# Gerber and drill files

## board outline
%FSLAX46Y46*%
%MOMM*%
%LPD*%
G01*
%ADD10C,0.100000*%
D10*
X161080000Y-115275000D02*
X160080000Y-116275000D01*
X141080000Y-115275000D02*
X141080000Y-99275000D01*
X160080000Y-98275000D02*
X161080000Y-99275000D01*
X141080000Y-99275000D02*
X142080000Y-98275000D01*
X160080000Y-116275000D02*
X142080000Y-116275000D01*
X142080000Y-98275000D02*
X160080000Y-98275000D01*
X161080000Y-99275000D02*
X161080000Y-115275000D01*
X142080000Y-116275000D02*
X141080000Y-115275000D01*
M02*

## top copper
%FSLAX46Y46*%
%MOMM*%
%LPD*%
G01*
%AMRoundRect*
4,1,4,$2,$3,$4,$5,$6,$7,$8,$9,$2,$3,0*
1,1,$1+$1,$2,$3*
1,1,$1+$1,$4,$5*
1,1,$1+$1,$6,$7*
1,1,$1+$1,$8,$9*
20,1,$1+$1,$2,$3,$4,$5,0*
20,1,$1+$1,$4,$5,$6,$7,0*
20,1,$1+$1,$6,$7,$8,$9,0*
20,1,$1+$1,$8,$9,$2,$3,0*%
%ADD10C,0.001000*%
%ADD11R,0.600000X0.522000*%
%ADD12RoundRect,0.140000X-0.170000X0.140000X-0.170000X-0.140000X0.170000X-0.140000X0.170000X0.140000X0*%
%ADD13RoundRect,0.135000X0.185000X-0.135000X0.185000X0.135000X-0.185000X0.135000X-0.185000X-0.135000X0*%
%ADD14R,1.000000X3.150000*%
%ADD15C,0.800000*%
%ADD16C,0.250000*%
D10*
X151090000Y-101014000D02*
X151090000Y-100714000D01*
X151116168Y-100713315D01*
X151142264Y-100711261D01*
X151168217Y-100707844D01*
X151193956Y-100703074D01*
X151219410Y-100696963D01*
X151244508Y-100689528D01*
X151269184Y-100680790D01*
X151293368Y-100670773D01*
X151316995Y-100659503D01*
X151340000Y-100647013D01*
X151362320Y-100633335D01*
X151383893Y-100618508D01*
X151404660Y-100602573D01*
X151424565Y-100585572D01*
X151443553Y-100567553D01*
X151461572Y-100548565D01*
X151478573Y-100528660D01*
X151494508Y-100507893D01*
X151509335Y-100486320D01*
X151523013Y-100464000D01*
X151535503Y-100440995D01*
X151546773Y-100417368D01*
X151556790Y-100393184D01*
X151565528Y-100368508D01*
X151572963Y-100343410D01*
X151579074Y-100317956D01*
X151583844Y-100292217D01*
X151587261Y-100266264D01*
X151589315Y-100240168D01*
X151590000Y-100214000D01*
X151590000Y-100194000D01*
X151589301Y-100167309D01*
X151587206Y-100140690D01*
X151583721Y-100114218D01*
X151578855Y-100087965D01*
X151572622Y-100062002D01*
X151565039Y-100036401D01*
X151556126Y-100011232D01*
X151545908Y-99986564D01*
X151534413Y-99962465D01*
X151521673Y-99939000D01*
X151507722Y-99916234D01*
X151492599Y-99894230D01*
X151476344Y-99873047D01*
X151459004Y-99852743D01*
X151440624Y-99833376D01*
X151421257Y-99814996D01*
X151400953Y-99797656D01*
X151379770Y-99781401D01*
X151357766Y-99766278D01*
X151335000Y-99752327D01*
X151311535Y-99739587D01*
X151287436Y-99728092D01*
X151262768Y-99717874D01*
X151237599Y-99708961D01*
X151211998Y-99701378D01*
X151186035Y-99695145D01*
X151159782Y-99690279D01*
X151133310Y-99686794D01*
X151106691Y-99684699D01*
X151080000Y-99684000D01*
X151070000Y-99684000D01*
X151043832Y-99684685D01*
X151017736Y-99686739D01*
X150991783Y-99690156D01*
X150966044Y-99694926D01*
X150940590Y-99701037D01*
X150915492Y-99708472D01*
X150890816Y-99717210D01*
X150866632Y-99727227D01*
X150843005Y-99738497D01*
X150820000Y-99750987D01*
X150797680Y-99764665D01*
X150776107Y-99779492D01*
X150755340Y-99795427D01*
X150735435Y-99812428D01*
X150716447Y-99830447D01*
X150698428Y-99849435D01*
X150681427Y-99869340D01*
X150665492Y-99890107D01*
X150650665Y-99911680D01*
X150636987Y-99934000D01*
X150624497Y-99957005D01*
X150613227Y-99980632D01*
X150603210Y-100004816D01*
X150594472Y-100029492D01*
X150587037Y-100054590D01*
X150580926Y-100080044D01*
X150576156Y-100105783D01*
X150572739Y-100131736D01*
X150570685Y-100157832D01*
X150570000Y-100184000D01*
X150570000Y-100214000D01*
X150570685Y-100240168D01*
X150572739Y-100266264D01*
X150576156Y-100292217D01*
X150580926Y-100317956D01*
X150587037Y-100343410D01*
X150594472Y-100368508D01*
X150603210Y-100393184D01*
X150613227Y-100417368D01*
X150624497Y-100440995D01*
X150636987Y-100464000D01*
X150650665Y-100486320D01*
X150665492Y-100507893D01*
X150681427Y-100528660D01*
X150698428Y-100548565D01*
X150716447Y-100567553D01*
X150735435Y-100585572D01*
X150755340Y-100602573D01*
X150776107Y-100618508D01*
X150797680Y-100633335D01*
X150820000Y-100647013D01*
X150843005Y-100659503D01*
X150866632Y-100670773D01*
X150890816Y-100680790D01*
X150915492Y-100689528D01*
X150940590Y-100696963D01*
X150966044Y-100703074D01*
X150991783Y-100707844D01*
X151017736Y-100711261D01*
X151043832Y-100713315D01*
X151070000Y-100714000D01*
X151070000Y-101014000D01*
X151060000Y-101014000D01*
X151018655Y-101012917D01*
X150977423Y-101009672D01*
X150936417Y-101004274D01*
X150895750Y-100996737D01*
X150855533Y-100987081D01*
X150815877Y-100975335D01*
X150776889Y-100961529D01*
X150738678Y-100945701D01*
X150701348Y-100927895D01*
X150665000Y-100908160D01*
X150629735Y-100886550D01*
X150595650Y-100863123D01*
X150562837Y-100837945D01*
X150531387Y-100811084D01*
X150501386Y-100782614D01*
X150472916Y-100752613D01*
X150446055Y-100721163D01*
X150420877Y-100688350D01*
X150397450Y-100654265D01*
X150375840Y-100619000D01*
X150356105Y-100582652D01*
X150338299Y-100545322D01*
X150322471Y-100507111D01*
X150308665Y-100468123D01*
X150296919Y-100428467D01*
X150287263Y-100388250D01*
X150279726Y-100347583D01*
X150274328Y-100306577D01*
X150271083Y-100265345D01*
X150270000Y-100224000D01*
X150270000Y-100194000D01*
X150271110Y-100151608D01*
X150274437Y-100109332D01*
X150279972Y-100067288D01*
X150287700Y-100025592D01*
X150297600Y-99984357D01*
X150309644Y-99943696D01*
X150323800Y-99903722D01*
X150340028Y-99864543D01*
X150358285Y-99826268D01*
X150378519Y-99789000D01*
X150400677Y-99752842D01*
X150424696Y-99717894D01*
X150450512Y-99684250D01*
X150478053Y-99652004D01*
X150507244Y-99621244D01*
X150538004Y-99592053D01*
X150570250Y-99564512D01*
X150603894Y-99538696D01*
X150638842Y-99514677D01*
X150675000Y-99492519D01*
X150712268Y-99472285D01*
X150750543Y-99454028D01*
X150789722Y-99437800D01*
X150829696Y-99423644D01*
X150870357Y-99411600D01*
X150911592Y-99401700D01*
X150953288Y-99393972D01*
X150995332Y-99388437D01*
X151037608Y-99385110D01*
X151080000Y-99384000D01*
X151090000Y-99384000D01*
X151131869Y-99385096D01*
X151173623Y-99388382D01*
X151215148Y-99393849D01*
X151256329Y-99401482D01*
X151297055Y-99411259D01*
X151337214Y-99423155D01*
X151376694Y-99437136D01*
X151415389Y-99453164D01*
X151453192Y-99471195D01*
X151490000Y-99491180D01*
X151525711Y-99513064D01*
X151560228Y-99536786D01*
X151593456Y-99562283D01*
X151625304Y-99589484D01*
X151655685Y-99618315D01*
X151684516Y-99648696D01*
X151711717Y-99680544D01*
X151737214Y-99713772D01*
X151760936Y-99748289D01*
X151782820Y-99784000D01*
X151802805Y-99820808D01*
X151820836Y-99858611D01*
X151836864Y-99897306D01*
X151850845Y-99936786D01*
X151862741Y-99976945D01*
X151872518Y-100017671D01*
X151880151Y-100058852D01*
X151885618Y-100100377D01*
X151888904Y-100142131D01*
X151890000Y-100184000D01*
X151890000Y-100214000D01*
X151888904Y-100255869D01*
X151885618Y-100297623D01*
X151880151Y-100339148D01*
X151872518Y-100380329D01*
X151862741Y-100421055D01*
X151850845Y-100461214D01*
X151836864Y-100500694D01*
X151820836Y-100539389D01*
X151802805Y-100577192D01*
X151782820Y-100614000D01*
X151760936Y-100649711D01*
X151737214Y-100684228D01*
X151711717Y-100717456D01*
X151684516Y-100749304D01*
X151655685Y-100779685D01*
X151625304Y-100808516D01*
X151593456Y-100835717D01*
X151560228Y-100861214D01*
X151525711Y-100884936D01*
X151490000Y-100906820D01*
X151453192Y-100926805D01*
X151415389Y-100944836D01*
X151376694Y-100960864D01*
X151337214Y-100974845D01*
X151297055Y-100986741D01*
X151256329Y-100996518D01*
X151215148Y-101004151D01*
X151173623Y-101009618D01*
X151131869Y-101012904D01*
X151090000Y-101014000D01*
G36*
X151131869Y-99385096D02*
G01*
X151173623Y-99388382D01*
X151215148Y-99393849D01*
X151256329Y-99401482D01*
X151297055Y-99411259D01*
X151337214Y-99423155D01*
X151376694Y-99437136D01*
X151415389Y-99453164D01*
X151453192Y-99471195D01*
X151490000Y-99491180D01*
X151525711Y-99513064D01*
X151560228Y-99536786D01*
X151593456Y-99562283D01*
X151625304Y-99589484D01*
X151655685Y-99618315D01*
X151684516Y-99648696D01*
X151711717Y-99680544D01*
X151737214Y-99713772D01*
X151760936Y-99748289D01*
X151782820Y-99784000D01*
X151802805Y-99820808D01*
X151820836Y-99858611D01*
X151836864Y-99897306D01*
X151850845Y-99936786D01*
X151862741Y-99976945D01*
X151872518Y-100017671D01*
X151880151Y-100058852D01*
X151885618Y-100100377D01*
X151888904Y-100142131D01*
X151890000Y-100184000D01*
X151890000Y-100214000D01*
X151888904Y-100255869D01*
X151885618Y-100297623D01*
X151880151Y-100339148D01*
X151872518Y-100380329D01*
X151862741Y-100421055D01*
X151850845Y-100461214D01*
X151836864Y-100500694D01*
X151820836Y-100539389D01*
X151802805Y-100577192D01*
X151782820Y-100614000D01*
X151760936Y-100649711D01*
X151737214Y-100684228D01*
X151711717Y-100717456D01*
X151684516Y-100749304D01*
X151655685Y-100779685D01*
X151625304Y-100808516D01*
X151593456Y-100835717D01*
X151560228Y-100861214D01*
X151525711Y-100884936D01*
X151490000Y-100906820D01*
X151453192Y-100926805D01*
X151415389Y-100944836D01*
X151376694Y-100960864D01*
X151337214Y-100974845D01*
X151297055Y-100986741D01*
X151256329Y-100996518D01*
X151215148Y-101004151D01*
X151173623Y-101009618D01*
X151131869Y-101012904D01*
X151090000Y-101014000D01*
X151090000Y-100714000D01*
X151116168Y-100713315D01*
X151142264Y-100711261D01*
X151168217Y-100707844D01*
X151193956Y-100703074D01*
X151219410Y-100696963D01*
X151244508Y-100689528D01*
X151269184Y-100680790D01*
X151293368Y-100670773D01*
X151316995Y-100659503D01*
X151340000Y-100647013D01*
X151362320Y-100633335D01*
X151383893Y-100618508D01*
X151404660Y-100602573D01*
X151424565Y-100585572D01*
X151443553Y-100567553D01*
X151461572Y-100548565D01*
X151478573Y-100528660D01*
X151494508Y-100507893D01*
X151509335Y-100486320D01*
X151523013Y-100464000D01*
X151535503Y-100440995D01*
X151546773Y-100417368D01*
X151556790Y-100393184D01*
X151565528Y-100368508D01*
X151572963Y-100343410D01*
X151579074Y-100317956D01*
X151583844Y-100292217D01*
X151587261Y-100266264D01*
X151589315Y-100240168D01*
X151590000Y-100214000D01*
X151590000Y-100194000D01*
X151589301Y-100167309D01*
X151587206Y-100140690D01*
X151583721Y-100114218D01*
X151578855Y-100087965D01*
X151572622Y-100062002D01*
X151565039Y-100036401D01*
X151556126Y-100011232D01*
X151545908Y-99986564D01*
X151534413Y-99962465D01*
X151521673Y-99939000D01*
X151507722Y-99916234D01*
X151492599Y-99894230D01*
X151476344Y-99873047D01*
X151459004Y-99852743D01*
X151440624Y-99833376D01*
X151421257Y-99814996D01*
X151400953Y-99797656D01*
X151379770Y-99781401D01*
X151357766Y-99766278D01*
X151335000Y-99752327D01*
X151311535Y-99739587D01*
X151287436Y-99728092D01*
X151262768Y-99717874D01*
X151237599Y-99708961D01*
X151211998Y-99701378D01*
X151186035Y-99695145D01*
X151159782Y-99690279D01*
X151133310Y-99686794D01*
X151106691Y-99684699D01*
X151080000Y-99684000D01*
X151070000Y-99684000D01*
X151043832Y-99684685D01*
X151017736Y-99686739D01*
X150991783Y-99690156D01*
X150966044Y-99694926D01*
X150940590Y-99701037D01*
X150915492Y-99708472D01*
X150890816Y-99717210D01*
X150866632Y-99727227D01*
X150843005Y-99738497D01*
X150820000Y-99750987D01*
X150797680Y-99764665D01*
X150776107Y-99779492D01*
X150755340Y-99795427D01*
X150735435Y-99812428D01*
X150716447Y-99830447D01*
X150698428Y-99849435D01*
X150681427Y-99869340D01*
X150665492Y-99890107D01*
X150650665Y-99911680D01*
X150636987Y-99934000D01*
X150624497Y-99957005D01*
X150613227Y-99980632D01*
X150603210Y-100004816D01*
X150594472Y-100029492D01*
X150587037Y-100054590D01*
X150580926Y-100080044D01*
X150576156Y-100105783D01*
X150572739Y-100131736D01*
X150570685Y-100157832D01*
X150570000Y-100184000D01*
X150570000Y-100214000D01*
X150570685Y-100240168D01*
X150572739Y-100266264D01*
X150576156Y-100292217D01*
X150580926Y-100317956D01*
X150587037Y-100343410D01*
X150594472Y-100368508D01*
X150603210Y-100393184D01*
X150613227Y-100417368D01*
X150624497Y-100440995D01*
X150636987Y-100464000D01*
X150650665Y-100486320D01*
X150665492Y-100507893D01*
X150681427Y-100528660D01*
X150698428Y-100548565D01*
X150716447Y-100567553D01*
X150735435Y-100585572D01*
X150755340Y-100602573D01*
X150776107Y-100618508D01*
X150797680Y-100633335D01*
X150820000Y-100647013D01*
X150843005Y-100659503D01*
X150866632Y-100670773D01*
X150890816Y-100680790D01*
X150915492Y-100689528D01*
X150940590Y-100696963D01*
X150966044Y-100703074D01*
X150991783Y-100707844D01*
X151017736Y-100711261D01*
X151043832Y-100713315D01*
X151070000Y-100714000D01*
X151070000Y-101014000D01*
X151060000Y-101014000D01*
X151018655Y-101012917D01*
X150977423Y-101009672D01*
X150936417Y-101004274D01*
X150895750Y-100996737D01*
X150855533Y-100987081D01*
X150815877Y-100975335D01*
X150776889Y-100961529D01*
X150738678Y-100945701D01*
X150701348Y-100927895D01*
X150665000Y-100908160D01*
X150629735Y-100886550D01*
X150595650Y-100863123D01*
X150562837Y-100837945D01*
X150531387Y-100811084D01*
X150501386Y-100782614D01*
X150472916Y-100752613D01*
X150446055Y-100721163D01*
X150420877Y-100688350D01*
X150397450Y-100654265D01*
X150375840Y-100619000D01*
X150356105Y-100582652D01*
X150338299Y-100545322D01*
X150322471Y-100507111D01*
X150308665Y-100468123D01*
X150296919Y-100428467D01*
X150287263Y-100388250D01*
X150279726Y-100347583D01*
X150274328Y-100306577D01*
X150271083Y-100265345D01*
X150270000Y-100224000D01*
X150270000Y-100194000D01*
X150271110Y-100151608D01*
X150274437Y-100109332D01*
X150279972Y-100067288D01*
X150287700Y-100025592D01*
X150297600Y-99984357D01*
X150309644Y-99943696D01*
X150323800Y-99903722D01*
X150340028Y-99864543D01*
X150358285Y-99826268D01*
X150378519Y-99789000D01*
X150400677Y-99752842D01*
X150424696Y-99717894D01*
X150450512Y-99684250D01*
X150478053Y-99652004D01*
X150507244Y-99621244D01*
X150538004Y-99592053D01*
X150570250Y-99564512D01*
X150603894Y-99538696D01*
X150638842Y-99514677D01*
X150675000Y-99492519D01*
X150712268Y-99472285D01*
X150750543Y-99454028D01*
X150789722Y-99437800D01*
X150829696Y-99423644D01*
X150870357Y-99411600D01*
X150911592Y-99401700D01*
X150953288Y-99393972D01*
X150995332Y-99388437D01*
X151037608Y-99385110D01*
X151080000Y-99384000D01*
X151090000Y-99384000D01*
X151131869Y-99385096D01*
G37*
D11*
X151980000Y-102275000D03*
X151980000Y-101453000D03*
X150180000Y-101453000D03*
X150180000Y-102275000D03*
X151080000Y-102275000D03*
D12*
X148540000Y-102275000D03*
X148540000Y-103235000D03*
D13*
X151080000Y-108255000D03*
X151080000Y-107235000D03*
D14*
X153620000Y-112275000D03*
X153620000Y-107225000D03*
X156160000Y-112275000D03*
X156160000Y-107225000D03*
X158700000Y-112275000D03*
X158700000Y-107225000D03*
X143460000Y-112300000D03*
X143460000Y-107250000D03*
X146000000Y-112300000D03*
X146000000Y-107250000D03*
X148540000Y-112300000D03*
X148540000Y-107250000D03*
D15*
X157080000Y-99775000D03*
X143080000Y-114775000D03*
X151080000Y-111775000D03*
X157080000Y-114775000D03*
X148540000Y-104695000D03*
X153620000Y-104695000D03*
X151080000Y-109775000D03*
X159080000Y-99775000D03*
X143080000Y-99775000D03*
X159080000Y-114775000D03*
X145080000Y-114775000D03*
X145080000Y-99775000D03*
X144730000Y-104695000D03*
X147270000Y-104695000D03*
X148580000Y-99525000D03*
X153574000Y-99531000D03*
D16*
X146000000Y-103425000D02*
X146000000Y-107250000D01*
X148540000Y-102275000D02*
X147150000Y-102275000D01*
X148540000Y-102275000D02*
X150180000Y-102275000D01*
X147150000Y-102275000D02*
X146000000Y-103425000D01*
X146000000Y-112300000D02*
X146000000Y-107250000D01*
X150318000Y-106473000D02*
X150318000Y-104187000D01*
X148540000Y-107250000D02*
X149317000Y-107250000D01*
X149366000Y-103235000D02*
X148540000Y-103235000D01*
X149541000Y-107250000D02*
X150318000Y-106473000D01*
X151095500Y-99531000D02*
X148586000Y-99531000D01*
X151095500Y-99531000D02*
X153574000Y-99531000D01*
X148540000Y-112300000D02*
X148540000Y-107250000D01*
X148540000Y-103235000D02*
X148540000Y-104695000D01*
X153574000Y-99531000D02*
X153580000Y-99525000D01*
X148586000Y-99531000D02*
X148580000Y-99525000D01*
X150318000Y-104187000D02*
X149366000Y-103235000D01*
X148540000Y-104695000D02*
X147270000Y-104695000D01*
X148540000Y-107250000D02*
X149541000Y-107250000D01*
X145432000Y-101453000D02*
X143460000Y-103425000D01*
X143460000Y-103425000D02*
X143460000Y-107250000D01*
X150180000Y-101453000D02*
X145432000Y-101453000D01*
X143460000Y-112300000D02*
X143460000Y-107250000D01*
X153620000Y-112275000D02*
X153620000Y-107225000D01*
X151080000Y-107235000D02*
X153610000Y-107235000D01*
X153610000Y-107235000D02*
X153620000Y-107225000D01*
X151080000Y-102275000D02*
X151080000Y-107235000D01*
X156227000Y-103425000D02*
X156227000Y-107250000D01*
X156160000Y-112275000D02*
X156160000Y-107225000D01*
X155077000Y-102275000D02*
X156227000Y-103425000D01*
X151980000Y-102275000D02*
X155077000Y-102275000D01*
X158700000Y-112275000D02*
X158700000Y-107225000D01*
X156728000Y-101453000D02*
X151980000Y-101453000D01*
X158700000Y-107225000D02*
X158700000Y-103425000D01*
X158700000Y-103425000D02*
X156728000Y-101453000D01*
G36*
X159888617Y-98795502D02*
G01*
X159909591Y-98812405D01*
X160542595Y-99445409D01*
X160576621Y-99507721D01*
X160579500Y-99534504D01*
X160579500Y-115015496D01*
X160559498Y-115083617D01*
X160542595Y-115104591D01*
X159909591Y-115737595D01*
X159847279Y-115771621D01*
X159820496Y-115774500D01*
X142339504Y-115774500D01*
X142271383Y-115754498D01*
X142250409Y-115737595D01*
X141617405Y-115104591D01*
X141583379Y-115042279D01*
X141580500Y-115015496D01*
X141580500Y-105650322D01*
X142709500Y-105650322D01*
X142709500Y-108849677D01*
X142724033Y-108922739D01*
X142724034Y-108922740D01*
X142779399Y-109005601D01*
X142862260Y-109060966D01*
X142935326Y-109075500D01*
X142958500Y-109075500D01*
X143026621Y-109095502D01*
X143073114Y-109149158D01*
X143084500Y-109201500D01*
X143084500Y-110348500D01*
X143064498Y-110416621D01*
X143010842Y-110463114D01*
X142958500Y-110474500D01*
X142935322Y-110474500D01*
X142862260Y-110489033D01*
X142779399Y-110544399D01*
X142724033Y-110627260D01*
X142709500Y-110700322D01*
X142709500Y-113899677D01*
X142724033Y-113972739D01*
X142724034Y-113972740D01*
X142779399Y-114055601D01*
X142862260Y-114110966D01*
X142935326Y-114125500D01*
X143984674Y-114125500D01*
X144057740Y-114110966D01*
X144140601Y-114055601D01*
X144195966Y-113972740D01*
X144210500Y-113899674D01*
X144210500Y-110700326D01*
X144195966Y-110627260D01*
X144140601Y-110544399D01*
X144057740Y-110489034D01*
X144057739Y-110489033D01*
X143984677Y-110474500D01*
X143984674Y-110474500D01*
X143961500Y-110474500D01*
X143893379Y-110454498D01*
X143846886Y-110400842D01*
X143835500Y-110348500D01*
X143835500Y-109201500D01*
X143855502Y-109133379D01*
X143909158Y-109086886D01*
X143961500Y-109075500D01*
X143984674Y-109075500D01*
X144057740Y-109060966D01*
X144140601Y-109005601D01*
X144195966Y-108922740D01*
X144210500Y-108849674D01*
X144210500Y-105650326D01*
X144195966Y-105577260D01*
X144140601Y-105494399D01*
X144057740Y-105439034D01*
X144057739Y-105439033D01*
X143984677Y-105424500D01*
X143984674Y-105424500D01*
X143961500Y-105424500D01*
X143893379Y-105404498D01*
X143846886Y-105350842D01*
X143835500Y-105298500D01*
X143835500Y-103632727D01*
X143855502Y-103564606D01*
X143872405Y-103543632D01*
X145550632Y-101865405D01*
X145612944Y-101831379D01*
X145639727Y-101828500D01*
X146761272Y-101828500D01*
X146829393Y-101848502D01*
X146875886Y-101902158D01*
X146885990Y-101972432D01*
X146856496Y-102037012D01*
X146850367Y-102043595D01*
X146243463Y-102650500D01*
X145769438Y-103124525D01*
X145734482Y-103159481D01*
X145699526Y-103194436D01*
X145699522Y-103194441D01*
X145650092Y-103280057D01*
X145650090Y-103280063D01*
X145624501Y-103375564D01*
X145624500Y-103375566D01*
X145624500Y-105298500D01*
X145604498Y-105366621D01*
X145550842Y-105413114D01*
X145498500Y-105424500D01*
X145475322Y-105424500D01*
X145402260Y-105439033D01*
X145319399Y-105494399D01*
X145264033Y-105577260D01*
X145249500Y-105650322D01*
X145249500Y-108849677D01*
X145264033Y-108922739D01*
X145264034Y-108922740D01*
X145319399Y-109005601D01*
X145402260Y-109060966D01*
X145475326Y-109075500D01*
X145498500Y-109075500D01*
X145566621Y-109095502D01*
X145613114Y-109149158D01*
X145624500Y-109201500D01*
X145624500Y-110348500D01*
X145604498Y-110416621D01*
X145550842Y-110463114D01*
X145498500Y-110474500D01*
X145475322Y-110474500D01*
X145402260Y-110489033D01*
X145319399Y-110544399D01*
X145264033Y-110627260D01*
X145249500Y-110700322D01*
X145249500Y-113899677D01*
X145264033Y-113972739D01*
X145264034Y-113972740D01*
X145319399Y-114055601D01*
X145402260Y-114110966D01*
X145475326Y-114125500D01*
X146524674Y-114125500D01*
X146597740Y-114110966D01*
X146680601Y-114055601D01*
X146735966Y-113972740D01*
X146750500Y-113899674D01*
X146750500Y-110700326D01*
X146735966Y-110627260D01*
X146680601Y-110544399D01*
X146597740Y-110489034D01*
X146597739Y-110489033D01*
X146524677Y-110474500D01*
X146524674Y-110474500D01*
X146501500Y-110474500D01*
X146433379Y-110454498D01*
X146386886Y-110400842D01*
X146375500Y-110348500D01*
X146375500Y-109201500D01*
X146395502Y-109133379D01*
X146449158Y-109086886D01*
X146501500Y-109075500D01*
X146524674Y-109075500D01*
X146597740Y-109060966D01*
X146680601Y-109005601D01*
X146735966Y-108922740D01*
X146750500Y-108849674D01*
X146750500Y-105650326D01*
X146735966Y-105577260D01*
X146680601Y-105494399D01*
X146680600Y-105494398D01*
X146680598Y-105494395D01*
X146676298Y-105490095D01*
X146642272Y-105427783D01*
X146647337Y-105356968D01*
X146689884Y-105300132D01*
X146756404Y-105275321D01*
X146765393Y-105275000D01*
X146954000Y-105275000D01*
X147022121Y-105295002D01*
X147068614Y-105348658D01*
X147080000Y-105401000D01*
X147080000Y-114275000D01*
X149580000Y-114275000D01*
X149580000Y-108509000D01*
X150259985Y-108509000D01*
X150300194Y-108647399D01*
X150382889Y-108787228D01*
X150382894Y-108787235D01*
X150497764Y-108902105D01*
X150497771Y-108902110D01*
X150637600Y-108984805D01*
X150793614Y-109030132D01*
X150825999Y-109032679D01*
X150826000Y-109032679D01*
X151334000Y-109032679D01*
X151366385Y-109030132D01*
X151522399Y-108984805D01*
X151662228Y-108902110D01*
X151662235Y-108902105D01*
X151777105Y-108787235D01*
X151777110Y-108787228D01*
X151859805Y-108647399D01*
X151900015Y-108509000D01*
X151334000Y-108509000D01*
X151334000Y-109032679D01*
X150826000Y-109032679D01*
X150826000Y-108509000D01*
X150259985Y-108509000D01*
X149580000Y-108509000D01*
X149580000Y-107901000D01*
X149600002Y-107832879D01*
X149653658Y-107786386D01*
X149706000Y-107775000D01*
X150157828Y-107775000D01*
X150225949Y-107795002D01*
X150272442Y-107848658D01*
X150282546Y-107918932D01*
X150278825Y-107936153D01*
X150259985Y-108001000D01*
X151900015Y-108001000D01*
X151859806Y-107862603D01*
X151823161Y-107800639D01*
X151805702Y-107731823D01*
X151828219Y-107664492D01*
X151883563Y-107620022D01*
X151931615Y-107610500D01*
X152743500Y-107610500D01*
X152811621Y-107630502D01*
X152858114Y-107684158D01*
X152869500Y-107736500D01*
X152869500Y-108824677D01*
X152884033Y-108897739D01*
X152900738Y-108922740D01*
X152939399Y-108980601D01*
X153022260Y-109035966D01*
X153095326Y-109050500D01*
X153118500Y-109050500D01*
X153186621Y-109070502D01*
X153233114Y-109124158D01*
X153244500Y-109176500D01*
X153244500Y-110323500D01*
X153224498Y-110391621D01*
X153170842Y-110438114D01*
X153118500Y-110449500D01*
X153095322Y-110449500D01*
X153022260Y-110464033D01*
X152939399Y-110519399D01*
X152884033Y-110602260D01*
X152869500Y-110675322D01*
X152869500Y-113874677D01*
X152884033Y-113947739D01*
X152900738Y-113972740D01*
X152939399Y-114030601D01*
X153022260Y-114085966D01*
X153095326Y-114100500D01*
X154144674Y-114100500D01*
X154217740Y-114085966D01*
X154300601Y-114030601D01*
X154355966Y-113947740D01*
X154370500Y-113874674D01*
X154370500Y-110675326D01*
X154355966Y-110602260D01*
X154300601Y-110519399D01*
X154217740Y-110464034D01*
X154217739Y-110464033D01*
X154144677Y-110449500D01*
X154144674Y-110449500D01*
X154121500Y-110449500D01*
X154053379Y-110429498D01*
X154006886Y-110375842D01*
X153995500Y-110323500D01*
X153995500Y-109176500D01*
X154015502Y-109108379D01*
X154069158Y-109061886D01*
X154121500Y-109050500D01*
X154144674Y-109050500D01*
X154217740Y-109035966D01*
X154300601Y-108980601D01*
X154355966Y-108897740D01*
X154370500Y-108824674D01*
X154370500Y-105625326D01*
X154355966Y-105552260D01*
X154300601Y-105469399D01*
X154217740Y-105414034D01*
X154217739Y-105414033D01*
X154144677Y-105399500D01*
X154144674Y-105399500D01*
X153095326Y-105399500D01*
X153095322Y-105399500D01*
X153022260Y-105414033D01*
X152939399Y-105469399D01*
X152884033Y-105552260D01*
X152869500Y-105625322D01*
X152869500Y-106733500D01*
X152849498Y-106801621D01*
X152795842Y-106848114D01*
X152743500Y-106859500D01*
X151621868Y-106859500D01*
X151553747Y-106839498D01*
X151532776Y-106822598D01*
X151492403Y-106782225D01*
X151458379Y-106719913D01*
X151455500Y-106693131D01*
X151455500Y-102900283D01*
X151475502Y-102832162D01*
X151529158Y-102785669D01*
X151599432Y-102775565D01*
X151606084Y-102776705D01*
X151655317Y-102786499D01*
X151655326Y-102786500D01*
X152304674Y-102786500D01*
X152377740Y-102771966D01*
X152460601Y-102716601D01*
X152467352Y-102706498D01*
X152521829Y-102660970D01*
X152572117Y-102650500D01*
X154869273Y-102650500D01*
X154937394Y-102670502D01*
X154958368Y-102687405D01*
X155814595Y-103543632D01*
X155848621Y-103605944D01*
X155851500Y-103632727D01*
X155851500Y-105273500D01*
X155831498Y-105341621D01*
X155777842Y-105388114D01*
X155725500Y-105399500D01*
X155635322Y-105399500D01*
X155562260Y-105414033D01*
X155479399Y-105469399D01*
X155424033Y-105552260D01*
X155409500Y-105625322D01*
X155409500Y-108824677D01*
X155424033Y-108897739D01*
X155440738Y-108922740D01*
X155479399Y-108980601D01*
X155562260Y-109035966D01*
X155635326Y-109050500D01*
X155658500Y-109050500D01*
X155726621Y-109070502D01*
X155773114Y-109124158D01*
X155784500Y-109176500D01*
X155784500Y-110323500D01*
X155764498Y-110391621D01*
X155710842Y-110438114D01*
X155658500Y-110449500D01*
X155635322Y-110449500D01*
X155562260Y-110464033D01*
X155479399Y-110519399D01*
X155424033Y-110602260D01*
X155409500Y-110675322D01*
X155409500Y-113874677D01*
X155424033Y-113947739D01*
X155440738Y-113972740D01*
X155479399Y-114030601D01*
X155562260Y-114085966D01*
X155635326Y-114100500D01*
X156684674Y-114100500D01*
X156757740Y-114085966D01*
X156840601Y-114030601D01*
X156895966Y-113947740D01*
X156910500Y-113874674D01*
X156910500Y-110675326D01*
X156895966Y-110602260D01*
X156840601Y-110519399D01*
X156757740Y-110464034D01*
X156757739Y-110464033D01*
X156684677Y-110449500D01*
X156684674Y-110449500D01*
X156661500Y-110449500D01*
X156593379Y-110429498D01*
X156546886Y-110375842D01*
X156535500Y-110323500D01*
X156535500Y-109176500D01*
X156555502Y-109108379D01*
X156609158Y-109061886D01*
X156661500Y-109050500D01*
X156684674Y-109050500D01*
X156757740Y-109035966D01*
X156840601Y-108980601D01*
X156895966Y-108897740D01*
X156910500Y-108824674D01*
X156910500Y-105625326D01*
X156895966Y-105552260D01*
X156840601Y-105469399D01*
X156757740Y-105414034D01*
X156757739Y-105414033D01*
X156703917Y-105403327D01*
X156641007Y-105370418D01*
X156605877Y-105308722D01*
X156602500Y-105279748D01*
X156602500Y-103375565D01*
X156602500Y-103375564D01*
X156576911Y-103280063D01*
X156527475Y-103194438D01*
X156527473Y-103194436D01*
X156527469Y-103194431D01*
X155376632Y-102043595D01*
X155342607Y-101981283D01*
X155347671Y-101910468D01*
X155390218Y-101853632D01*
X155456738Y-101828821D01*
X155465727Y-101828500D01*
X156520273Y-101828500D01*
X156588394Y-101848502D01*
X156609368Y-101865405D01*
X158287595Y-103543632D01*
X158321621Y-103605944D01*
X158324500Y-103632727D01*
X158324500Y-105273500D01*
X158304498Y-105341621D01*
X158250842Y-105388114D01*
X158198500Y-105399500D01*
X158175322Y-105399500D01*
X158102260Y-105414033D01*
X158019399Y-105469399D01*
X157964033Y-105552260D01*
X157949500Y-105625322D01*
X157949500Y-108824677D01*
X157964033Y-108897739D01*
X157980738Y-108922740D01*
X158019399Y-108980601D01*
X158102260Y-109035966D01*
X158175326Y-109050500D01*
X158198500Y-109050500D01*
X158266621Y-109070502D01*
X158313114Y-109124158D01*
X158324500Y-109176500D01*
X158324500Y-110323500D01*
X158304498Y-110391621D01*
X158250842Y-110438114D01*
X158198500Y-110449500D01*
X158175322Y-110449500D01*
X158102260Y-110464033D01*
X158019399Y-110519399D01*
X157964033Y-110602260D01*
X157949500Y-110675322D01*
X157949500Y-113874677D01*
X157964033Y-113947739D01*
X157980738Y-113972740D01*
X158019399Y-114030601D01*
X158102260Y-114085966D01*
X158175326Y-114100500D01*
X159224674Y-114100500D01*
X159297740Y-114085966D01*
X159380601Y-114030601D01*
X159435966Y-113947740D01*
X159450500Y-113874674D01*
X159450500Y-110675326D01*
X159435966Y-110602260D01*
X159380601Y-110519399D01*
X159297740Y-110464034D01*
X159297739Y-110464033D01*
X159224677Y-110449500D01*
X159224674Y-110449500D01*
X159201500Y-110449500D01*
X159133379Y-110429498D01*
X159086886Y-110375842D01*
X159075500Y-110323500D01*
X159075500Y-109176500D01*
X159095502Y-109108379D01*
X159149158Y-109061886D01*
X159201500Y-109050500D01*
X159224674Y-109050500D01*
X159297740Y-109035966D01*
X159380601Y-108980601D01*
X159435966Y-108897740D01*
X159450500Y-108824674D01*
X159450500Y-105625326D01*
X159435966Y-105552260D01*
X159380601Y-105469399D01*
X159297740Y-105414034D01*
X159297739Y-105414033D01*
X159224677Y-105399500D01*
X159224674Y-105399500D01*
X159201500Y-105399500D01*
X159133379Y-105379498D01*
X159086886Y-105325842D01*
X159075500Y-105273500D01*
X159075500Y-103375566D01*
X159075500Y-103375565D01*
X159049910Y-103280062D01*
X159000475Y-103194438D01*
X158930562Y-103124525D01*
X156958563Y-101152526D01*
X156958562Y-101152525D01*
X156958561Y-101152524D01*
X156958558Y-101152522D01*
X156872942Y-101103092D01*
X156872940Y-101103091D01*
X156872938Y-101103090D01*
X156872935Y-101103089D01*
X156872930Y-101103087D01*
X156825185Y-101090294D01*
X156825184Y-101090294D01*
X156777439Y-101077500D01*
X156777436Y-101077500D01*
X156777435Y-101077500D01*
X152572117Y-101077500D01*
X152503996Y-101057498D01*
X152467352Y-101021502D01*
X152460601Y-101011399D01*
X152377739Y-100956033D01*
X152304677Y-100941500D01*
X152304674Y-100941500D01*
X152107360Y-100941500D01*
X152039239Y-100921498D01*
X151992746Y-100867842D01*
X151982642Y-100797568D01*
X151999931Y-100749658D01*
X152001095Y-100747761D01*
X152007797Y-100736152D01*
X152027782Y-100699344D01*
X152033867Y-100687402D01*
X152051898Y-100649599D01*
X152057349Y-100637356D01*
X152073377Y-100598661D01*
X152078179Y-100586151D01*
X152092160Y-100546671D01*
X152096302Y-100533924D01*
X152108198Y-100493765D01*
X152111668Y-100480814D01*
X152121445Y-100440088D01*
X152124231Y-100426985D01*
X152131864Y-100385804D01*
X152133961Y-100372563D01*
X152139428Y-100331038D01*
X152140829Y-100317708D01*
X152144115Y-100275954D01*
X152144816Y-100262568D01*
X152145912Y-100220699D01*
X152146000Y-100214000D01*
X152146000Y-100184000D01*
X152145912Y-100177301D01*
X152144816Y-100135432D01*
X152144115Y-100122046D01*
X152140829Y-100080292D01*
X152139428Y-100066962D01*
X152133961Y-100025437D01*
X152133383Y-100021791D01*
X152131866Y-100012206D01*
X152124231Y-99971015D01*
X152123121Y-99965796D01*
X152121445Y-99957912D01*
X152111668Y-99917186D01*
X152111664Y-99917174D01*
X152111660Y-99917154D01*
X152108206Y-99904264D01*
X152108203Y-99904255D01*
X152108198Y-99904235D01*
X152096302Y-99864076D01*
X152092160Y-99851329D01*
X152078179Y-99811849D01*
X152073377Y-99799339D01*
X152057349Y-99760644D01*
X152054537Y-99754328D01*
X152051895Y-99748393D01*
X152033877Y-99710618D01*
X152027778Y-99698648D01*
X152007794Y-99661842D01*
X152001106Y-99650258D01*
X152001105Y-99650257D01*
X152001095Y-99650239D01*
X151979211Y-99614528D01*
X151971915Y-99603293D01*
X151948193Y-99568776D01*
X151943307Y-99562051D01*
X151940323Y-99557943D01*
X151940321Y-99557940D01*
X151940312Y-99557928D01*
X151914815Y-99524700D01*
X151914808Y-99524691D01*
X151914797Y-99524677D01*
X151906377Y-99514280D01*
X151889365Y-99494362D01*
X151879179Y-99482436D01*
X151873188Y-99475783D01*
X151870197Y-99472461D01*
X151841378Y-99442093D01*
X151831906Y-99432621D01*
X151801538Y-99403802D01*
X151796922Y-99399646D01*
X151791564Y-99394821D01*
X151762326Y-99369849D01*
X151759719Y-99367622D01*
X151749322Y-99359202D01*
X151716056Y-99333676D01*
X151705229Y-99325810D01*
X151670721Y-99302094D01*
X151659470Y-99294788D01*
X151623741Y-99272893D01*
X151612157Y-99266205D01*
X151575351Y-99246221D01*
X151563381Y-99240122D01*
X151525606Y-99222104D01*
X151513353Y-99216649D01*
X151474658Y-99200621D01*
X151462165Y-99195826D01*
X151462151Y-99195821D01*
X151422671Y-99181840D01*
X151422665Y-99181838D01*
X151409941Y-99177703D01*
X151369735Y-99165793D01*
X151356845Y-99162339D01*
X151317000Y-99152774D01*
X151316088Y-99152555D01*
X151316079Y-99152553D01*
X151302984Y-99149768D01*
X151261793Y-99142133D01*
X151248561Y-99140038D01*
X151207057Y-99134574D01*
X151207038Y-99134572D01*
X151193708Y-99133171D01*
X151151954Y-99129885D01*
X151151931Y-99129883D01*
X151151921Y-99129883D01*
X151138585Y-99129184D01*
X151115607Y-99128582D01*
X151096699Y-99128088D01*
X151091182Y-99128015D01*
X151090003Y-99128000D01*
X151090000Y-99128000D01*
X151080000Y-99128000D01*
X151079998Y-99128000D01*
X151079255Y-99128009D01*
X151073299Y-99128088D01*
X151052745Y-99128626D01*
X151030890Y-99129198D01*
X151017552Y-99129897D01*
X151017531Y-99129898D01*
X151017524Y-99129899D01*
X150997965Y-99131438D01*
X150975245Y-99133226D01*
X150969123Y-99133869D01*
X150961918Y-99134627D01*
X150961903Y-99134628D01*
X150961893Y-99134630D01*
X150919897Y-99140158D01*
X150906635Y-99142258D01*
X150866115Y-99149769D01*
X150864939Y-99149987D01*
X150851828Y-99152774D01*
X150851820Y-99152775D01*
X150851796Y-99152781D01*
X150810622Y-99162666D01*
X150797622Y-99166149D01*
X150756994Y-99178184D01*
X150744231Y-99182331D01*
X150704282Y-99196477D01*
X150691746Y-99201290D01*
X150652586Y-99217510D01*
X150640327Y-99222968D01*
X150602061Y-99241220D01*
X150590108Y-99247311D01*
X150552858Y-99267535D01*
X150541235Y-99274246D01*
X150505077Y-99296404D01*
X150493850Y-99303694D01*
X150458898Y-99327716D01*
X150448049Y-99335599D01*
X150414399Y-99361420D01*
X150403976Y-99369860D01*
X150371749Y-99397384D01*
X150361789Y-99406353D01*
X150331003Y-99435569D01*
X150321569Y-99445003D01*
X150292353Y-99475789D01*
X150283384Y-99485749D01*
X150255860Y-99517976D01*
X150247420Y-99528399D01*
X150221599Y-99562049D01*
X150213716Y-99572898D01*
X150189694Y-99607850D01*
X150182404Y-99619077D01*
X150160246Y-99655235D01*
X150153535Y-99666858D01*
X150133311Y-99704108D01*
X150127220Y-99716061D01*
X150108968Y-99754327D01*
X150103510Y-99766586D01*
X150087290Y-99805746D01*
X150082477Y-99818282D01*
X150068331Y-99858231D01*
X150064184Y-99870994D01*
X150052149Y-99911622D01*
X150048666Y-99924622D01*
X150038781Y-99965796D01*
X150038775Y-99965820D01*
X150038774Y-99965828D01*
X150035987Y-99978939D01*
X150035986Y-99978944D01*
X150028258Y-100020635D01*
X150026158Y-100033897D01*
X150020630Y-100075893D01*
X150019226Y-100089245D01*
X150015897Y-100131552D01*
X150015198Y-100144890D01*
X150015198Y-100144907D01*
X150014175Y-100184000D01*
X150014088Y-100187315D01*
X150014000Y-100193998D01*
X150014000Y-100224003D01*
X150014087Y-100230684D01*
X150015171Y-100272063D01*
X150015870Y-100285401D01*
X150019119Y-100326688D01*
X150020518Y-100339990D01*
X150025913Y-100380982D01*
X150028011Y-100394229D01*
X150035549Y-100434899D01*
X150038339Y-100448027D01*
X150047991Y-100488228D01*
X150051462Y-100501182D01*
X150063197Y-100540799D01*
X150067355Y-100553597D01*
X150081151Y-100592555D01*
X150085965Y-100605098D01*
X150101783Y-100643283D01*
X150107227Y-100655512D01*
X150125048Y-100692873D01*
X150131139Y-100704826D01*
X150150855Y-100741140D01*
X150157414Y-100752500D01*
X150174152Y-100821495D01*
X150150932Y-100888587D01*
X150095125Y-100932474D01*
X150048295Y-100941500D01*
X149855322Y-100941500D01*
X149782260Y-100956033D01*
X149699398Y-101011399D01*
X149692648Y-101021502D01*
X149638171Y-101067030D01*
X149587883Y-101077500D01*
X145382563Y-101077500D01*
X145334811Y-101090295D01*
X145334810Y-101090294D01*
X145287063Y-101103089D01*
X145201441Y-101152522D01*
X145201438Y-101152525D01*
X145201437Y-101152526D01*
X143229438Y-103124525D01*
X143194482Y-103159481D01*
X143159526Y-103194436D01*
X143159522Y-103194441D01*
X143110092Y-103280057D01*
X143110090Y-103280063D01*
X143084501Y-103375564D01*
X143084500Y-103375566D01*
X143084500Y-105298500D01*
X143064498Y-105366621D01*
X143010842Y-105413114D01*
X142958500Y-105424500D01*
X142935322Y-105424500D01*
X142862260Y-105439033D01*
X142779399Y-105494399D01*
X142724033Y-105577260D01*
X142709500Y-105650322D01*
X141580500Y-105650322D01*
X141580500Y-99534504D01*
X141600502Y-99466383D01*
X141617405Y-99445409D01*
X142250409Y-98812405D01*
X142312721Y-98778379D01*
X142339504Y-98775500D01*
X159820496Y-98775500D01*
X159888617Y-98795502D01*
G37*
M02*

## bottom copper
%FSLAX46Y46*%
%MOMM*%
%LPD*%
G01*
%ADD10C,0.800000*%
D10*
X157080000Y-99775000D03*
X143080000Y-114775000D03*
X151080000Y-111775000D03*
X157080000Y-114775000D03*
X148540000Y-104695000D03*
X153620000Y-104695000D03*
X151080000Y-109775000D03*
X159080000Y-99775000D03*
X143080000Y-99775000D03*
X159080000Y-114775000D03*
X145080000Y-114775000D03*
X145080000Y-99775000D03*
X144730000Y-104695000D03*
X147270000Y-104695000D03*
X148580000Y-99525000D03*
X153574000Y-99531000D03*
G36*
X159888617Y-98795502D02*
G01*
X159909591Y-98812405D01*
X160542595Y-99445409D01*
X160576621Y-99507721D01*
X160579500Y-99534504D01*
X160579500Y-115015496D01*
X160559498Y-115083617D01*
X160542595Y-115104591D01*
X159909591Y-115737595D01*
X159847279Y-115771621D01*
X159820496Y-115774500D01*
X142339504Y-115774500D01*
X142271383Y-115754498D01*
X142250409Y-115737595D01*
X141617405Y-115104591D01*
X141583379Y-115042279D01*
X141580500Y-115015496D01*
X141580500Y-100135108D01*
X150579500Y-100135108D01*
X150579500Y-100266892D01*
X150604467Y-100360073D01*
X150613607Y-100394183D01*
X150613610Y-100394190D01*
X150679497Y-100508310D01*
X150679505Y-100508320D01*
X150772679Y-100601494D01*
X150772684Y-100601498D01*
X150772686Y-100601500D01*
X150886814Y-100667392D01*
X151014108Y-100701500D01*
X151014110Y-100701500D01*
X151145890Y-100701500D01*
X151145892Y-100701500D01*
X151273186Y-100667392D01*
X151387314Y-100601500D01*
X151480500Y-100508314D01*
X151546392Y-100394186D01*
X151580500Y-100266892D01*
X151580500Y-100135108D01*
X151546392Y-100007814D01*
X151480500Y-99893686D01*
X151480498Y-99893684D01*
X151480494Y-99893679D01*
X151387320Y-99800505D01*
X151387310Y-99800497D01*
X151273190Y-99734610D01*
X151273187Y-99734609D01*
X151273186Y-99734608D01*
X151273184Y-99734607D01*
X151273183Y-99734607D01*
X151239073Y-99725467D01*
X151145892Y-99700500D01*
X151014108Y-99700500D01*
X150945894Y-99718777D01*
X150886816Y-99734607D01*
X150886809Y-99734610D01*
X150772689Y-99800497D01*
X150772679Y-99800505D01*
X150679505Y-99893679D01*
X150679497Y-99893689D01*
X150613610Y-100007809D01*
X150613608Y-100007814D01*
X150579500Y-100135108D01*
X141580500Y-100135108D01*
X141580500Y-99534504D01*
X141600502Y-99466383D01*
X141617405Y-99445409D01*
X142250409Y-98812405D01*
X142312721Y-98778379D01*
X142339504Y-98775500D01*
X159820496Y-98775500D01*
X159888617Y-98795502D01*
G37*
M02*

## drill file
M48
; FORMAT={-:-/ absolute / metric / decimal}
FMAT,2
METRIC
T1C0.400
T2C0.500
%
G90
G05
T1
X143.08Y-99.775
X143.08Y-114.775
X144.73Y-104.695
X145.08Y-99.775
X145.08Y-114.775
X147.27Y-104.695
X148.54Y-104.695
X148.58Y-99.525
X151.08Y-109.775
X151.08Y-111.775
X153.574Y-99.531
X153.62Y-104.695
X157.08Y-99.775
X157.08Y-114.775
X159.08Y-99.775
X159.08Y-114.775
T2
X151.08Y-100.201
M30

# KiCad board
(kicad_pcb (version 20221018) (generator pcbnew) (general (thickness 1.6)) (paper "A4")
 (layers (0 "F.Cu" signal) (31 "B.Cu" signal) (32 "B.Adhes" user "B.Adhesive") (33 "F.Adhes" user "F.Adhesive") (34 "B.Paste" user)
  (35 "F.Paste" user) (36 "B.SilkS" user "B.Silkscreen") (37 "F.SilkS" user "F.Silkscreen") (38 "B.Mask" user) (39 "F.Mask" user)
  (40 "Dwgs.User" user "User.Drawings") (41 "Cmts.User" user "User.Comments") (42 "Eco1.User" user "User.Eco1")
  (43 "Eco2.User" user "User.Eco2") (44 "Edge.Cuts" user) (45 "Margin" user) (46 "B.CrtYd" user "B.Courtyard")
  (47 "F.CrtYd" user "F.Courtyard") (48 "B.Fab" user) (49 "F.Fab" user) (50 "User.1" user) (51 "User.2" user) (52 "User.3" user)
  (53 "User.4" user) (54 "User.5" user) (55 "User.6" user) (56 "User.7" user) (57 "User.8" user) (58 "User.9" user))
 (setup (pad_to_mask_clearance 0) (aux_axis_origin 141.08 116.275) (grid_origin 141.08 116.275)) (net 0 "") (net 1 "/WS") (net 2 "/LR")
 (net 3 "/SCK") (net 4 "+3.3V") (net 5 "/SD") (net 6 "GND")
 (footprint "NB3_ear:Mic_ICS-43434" (layer "F.Cu") (at 151.08 100.914 180)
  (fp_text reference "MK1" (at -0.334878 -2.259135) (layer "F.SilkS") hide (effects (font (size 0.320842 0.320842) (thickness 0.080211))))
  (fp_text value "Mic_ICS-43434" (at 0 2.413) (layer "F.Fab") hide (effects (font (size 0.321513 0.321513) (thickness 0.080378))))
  (fp_poly
   (pts (xy -0.01 -0.1) (xy -0.01 0.2) (xy -0.036168 0.200685) (xy -0.062264 0.202739) (xy -0.088217 0.206156) (xy -0.113956 0.210926)
    (xy -0.13941 0.217037) (xy -0.164508 0.224472) (xy -0.189184 0.23321) (xy -0.213368 0.243227) (xy -0.236995 0.254497)
    (xy -0.26 0.266987) (xy -0.28232 0.280665) (xy -0.303893 0.295492) (xy -0.32466 0.311427) (xy -0.344565 0.328428)
    (xy -0.363553 0.346447) (xy -0.381572 0.365435) (xy -0.398573 0.38534) (xy -0.414508 0.406107) (xy -0.429335 0.42768)
    (xy -0.443013 0.45) (xy -0.455503 0.473005) (xy -0.466773 0.496632) (xy -0.47679 0.520816) (xy -0.485528 0.545492)
    (xy -0.492963 0.57059) (xy -0.499074 0.596044) (xy -0.503844 0.621783) (xy -0.507261 0.647736) (xy -0.509315 0.673832) (xy -0.51 0.7)
    (xy -0.51 0.72) (xy -0.509301 0.746691) (xy -0.507206 0.77331) (xy -0.503721 0.799782) (xy -0.498855 0.826035) (xy -0.492622 0.851998)
    (xy -0.485039 0.877599) (xy -0.476126 0.902768) (xy -0.465908 0.927436) (xy -0.454413 0.951535) (xy -0.441673 0.975)
    (xy -0.427722 0.997766) (xy -0.412599 1.01977) (xy -0.396344 1.040953) (xy -0.379004 1.061257) (xy -0.360624 1.080624)
    (xy -0.341257 1.099004) (xy -0.320953 1.116344) (xy -0.29977 1.132599) (xy -0.277766 1.147722) (xy -0.255 1.161673)
    (xy -0.231535 1.174413) (xy -0.207436 1.185908) (xy -0.182768 1.196126) (xy -0.157599 1.205039) (xy -0.131998 1.212622)
    (xy -0.106035 1.218855) (xy -0.079782 1.223721) (xy -0.05331 1.227206) (xy -0.026691 1.229301) (xy 0 1.23) (xy 0.01 1.23)
    (xy 0.036168 1.229315) (xy 0.062264 1.227261) (xy 0.088217 1.223844) (xy 0.113956 1.219074) (xy 0.13941 1.212963) (xy 0.164508 1.205528)
    (xy 0.189184 1.19679) (xy 0.213368 1.186773) (xy 0.236995 1.175503) (xy 0.26 1.163013) (xy 0.28232 1.149335) (xy 0.303893 1.134508)
    (xy 0.32466 1.118573) (xy 0.344565 1.101572) (xy 0.363553 1.083553) (xy 0.381572 1.064565) (xy 0.398573 1.04466) (xy 0.414508 1.023893)
    (xy 0.429335 1.00232) (xy 0.443013 0.98) (xy 0.455503 0.956995) (xy 0.466773 0.933368) (xy 0.47679 0.909184) (xy 0.485528 0.884508)
    (xy 0.492963 0.85941) (xy 0.499074 0.833956) (xy 0.503844 0.808217) (xy 0.507261 0.782264) (xy 0.509315 0.756168) (xy 0.51 0.73)
    (xy 0.51 0.7) (xy 0.509315 0.673832) (xy 0.507261 0.647736) (xy 0.503844 0.621783) (xy 0.499074 0.596044) (xy 0.492963 0.57059)
    (xy 0.485528 0.545492) (xy 0.47679 0.520816) (xy 0.466773 0.496632) (xy 0.455503 0.473005) (xy 0.443013 0.45) (xy 0.429335 0.42768)
    (xy 0.414508 0.406107) (xy 0.398573 0.38534) (xy 0.381572 0.365435) (xy 0.363553 0.346447) (xy 0.344565 0.328428) (xy 0.32466 0.311427)
    (xy 0.303893 0.295492) (xy 0.28232 0.280665) (xy 0.26 0.266987) (xy 0.236995 0.254497) (xy 0.213368 0.243227) (xy 0.189184 0.23321)
    (xy 0.164508 0.224472) (xy 0.13941 0.217037) (xy 0.113956 0.210926) (xy 0.088217 0.206156) (xy 0.062264 0.202739) (xy 0.036168 0.200685)
    (xy 0.01 0.2) (xy 0.01 -0.1) (xy 0.02 -0.1) (xy 0.061345 -0.098917) (xy 0.102577 -0.095672) (xy 0.143583 -0.090274)
    (xy 0.18425 -0.082737) (xy 0.224467 -0.073081) (xy 0.264123 -0.061335) (xy 0.303111 -0.047529) (xy 0.341322 -0.031701)
    (xy 0.378652 -0.013895) (xy 0.415 0.00584) (xy 0.450265 0.02745) (xy 0.48435 0.050877) (xy 0.517163 0.076055) (xy 0.548613 0.102916)
    (xy 0.578614 0.131386) (xy 0.607084 0.161387) (xy 0.633945 0.192837) (xy 0.659123 0.22565) (xy 0.68255 0.259735) (xy 0.70416 0.295)
    (xy 0.723895 0.331348) (xy 0.741701 0.368678) (xy 0.757529 0.406889) (xy 0.771335 0.445877) (xy 0.783081 0.485533) (xy 0.792737 0.52575)
    (xy 0.800274 0.566417) (xy 0.805672 0.607423) (xy 0.808917 0.648655) (xy 0.81 0.69) (xy 0.81 0.72) (xy 0.80889 0.762392)
    (xy 0.805563 0.804668) (xy 0.800028 0.846712) (xy 0.7923 0.888408) (xy 0.7824 0.929643) (xy 0.770356 0.970304) (xy 0.7562 1.010278)
    (xy 0.739972 1.049457) (xy 0.721715 1.087732) (xy 0.701481 1.125) (xy 0.679323 1.161158) (xy 0.655304 1.196106) (xy 0.629488 1.22975)
    (xy 0.601947 1.261996) (xy 0.572756 1.292756) (xy 0.541996 1.321947) (xy 0.50975 1.349488) (xy 0.476106 1.375304) (xy 0.441158 1.399323)
    (xy 0.405 1.421481) (xy 0.367732 1.441715) (xy 0.329457 1.459972) (xy 0.290278 1.4762) (xy 0.250304 1.490356) (xy 0.209643 1.5024)
    (xy 0.168408 1.5123) (xy 0.126712 1.520028) (xy 0.084668 1.525563) (xy 0.042392 1.52889) (xy 0 1.53) (xy -0.01 1.53)
    (xy -0.051869 1.528904) (xy -0.093623 1.525618) (xy -0.135148 1.520151) (xy -0.176329 1.512518) (xy -0.217055 1.502741)
    (xy -0.257214 1.490845) (xy -0.296694 1.476864) (xy -0.335389 1.460836) (xy -0.373192 1.442805) (xy -0.41 1.42282)
    (xy -0.445711 1.400936) (xy -0.480228 1.377214) (xy -0.513456 1.351717) (xy -0.545304 1.324516) (xy -0.575685 1.295685)
    (xy -0.604516 1.265304) (xy -0.631717 1.233456) (xy -0.657214 1.200228) (xy -0.680936 1.165711) (xy -0.70282 1.13)
    (xy -0.722805 1.093192) (xy -0.740836 1.055389) (xy -0.756864 1.016694) (xy -0.770845 0.977214) (xy -0.782741 0.937055)
    (xy -0.792518 0.896329) (xy -0.800151 0.855148) (xy -0.805618 0.813623) (xy -0.808904 0.771869) (xy -0.81 0.73) (xy -0.81 0.7)
    (xy -0.808904 0.658131) (xy -0.805618 0.616377) (xy -0.800151 0.574852) (xy -0.792518 0.533671) (xy -0.782741 0.492945)
    (xy -0.770845 0.452786) (xy -0.756864 0.413306) (xy -0.740836 0.374611) (xy -0.722805 0.336808) (xy -0.70282 0.3)
    (xy -0.680936 0.264289) (xy -0.657214 0.229772) (xy -0.631717 0.196544) (xy -0.604516 0.164696) (xy -0.575685 0.134315)
    (xy -0.545304 0.105484) (xy -0.513456 0.078283) (xy -0.480228 0.052786) (xy -0.445711 0.029064) (xy -0.41 0.00718)
    (xy -0.373192 -0.012805) (xy -0.335389 -0.030836) (xy -0.296694 -0.046864) (xy -0.257214 -0.060845) (xy -0.217055 -0.072741)
    (xy -0.176329 -0.082518) (xy -0.135148 -0.090151) (xy -0.093623 -0.095618) (xy -0.051869 -0.098904) (xy -0.01 -0.1))
   (stroke (width 0.001) (type solid)) (fill solid) (layer "F.Cu"))
  (pad "" np_thru_hole circle (at 0 0.713 180) (size 0.5 0.5) (drill 0.5) (layers "*.Cu" "*.Mask"))
  (pad "1" smd rect (at -0.9 -1.361 180) (size 0.6 0.522) (layers "F.Cu" "F.Mask") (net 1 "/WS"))
  (pad "2" smd rect (at -0.9 -0.539 180) (size 0.6 0.522) (layers "F.Cu" "F.Mask") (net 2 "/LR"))
  (pad "4" smd rect (at 0.9 -0.539 180) (size 0.6 0.522) (layers "F.Cu" "F.Mask") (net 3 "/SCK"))
  (pad "5" smd rect (at 0.9 -1.361 180) (size 0.6 0.522) (layers "F.Cu" "F.Mask") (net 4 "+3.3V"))
  (pad "6" smd rect (at 0 -1.361 180) (size 0.6 0.522) (layers "F.Cu" "F.Mask") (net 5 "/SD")))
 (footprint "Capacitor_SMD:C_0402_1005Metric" (layer "F.Cu") (at 148.54 102.755 -90)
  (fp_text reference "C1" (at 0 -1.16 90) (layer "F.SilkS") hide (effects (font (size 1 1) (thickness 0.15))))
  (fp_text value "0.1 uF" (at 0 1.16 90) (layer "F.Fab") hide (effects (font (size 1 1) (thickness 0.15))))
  (pad "1" smd roundrect (at -0.48 0 270) (size 0.56 0.62) (layers "F.Cu" "F.Paste" "F.Mask") (roundrect_rratio 0.25) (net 4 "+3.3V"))
  (pad "2" smd roundrect (at 0.48 0 270) (size 0.56 0.62) (layers "F.Cu" "F.Paste" "F.Mask") (roundrect_rratio 0.25) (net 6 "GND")))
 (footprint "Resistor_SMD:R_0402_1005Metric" (layer "F.Cu") (at 151.08 107.745 90)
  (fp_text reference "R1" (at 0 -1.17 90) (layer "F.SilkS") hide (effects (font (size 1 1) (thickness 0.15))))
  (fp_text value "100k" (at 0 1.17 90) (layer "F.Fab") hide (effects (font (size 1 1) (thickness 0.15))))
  (pad "1" smd roundrect (at -0.51 0 90) (size 0.54 0.64) (layers "F.Cu" "F.Paste" "F.Mask") (roundrect_rratio 0.25) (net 6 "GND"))
  (pad "2" smd roundrect (at 0.51 0 90) (size 0.54 0.64) (layers "F.Cu" "F.Paste" "F.Mask") (roundrect_rratio 0.25) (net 5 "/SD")))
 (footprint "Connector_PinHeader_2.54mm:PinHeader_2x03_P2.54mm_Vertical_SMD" (layer "F.Cu") (at 156.16 109.75 90)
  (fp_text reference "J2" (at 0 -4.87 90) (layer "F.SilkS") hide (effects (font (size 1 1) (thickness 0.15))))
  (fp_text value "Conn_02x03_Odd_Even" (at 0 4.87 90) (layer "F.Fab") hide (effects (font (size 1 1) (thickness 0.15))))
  (pad "1" smd rect (at -2.525 -2.54 90) (size 3.15 1) (layers "F.Cu" "F.Paste" "F.Mask") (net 5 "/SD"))
  (pad "2" smd rect (at 2.525 -2.54 90) (size 3.15 1) (layers "F.Cu" "F.Paste" "F.Mask") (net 5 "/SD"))
  (pad "3" smd rect (at -2.525 0 90) (size 3.15 1) (layers "F.Cu" "F.Paste" "F.Mask") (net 1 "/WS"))
  (pad "4" smd rect (at 2.525 0 90) (size 3.15 1) (layers "F.Cu" "F.Paste" "F.Mask") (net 1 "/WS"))
  (pad "5" smd rect (at -2.525 2.54 90) (size 3.15 1) (layers "F.Cu" "F.Paste" "F.Mask") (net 2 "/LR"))
  (pad "6" smd rect (at 2.525 2.54 90) (size 3.15 1) (layers "F.Cu" "F.Paste" "F.Mask") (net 2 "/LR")))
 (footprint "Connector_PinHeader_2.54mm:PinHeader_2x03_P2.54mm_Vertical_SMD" (layer "F.Cu") (at 146 109.775 90)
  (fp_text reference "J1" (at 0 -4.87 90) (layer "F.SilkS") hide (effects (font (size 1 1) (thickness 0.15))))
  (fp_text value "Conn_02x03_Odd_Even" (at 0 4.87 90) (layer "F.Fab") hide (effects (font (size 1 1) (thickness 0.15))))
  (pad "1" smd rect (at -2.525 -2.54 90) (size 3.15 1) (layers "F.Cu" "F.Paste" "F.Mask") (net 3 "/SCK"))
  (pad "2" smd rect (at 2.525 -2.54 90) (size 3.15 1) (layers "F.Cu" "F.Paste" "F.Mask") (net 3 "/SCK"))
  (pad "3" smd rect (at -2.525 0 90) (size 3.15 1) (layers "F.Cu" "F.Paste" "F.Mask") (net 4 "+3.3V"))
  (pad "4" smd rect (at 2.525 0 90) (size 3.15 1) (layers "F.Cu" "F.Paste" "F.Mask") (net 4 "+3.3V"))
  (pad "5" smd rect (at -2.525 2.54 90) (size 3.15 1) (layers "F.Cu" "F.Paste" "F.Mask") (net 6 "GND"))
  (pad "6" smd rect (at 2.525 2.54 90) (size 3.15 1) (layers "F.Cu" "F.Paste" "F.Mask") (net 6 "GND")))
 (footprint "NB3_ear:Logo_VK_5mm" (layer "B.Cu") (at 151.08 107.275 180)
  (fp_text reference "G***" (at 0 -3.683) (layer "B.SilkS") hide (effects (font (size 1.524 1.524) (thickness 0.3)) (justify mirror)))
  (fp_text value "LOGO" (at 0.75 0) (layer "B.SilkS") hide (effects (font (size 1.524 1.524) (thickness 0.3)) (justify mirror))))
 (gr_line (start 161.08 115.275) (end 160.08 116.275) (stroke (width 0.1) (type default)) (layer "Edge.Cuts"))
 (gr_line (start 141.08 115.275) (end 141.08 99.275) (stroke (width 0.1) (type default)) (layer "Edge.Cuts"))
 (gr_line (start 160.08 98.275) (end 161.08 99.275) (stroke (width 0.1) (type default)) (layer "Edge.Cuts"))
 (gr_line (start 141.08 99.275) (end 142.08 98.275) (stroke (width 0.1) (type default)) (layer "Edge.Cuts"))
 (gr_line (start 160.08 116.275) (end 142.08 116.275) (stroke (width 0.1) (type default)) (layer "Edge.Cuts"))
 (gr_line (start 142.08 98.275) (end 160.08 98.275) (stroke (width 0.1) (type default)) (layer "Edge.Cuts"))
 (gr_line (start 161.08 99.275) (end 161.08 115.275) (stroke (width 0.1) (type default)) (layer "Edge.Cuts"))
 (gr_line (start 142.08 116.275) (end 141.08 115.275) (stroke (width 0.1) (type default)) (layer "Edge.Cuts"))
 (segment (start 146 103.425) (end 146 107.25) (width 0.25) (layer "F.Cu") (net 4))
 (segment (start 148.54 102.275) (end 147.15 102.275) (width 0.25) (layer "F.Cu") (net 4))
 (segment (start 148.54 102.275) (end 150.18 102.275) (width 0.25) (layer "F.Cu") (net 4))
 (segment (start 147.15 102.275) (end 146 103.425) (width 0.25) (layer "F.Cu") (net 4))
 (segment (start 146 112.3) (end 146 107.25) (width 0.25) (layer "F.Cu") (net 4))
 (segment (start 150.318 106.473) (end 150.318 104.187) (width 0.25) (layer "F.Cu") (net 6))
 (segment (start 148.54 107.25) (end 149.317 107.25) (width 0.25) (layer "F.Cu") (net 6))
 (segment (start 149.366 103.235) (end 148.54 103.235) (width 0.25) (layer "F.Cu") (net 6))
 (segment (start 149.541 107.25) (end 150.318 106.473) (width 0.25) (layer "F.Cu") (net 6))
 (segment (start 151.0955 99.531) (end 148.586 99.531) (width 0.25) (layer "F.Cu") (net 6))
 (segment (start 151.0955 99.531) (end 153.574 99.531) (width 0.25) (layer "F.Cu") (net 6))
 (segment (start 148.54 112.3) (end 148.54 107.25) (width 0.25) (layer "F.Cu") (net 6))
 (segment (start 148.54 103.235) (end 148.54 104.695) (width 0.25) (layer "F.Cu") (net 6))
 (segment (start 153.574 99.531) (end 153.58 99.525) (width 0.25) (layer "F.Cu") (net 6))
 (segment (start 148.586 99.531) (end 148.58 99.525) (width 0.25) (layer "F.Cu") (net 6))
 (segment (start 150.318 104.187) (end 149.366 103.235) (width 0.25) (layer "F.Cu") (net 6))
 (segment (start 148.54 104.695) (end 147.27 104.695) (width 0.25) (layer "F.Cu") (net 6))
 (segment (start 148.54 107.25) (end 149.541 107.25) (width 0.25) (layer "F.Cu") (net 6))
 (via (at 157.08 99.775) (size 0.8) (drill 0.4) (layers "F.Cu" "B.Cu") (free) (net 6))
 (via (at 143.08 114.775) (size 0.8) (drill 0.4) (layers "F.Cu" "B.Cu") (free) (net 6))
 (via (at 151.08 111.775) (size 0.8) (drill 0.4) (layers "F.Cu" "B.Cu") (free) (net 6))
 (via (at 157.08 114.775) (size 0.8) (drill 0.4) (layers "F.Cu" "B.Cu") (free) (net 6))
 (via (at 148.54 104.695) (size 0.8) (drill 0.4) (layers "F.Cu" "B.Cu") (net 6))
 (via (at 153.62 104.695) (size 0.8) (drill 0.4) (layers "F.Cu" "B.Cu") (free) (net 6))
 (via (at 151.08 109.775) (size 0.8) (drill 0.4) (layers "F.Cu" "B.Cu") (free) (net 6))
 (via (at 159.08 99.775) (size 0.8) (drill 0.4) (layers "F.Cu" "B.Cu") (free) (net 6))
 (via (at 143.08 99.775) (size 0.8) (drill 0.4) (layers "F.Cu" "B.Cu") (free) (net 6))
 (via (at 159.08 114.775) (size 0.8) (drill 0.4) (layers "F.Cu" "B.Cu") (free) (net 6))
 (via (at 145.08 114.775) (size 0.8) (drill 0.4) (layers "F.Cu" "B.Cu") (free) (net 6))
 (via (at 145.08 99.775) (size 0.8) (drill 0.4) (layers "F.Cu" "B.Cu") (free) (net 6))
 (via (at 144.73 104.695) (size 0.8) (drill 0.4) (layers "F.Cu" "B.Cu") (free) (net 6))
 (via (at 147.27 104.695) (size 0.8) (drill 0.4) (layers "F.Cu" "B.Cu") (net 6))
 (via (at 148.58 99.525) (size 0.8) (drill 0.4) (layers "F.Cu" "B.Cu") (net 6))
 (via (at 153.574 99.531) (size 0.8) (drill 0.4) (layers "F.Cu" "B.Cu") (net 6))
 (segment (start 145.432 101.453) (end 143.46 103.425) (width 0.25) (layer "F.Cu") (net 3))
 (segment (start 143.46 103.425) (end 143.46 107.25) (width 0.25) (layer "F.Cu") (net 3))
 (segment (start 150.18 101.453) (end 145.432 101.453) (width 0.25) (layer "F.Cu") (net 3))
 (segment (start 143.46 112.3) (end 143.46 107.25) (width 0.25) (layer "F.Cu") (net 3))
 (segment (start 153.62 112.275) (end 153.62 107.225) (width 0.25) (layer "F.Cu") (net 5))
 (segment (start 151.08 107.235) (end 153.61 107.235) (width 0.25) (layer "F.Cu") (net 5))
 (segment (start 153.61 107.235) (end 153.62 107.225) (width 0.25) (layer "F.Cu") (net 5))
 (segment (start 151.08 102.275) (end 151.08 107.235) (width 0.25) (layer "F.Cu") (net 5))
 (segment (start 156.227 103.425) (end 156.227 107.25) (width 0.25) (layer "F.Cu") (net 1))
 (segment (start 156.16 112.275) (end 156.16 107.225) (width 0.25) (layer "F.Cu") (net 1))
 (segment (start 155.077 102.275) (end 156.227 103.425) (width 0.25) (layer "F.Cu") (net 1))
 (segment (start 151.98 102.275) (end 155.077 102.275) (width 0.25) (layer "F.Cu") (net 1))
 (segment (start 158.7 112.275) (end 158.7 107.225) (width 0.25) (layer "F.Cu") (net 2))
 (segment (start 156.728 101.453) (end 151.98 101.453) (width 0.25) (layer "F.Cu") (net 2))
 (segment (start 158.7 107.225) (end 158.7 103.425) (width 0.25) (layer "F.Cu") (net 2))
 (segment (start 158.7 103.425) (end 156.728 101.453) (width 0.25) (layer "F.Cu") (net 2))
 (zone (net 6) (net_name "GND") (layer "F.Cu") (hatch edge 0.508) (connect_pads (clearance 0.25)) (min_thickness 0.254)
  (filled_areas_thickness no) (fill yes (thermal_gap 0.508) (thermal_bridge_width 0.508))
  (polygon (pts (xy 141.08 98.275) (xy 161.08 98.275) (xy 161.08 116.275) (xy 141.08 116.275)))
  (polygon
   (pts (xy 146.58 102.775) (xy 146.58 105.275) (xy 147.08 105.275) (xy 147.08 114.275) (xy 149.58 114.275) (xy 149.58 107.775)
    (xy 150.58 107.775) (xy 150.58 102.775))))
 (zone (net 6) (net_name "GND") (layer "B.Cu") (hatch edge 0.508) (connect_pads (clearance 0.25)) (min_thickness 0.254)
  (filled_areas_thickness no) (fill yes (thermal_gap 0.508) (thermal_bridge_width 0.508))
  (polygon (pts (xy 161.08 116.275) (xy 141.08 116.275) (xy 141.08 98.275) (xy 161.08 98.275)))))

